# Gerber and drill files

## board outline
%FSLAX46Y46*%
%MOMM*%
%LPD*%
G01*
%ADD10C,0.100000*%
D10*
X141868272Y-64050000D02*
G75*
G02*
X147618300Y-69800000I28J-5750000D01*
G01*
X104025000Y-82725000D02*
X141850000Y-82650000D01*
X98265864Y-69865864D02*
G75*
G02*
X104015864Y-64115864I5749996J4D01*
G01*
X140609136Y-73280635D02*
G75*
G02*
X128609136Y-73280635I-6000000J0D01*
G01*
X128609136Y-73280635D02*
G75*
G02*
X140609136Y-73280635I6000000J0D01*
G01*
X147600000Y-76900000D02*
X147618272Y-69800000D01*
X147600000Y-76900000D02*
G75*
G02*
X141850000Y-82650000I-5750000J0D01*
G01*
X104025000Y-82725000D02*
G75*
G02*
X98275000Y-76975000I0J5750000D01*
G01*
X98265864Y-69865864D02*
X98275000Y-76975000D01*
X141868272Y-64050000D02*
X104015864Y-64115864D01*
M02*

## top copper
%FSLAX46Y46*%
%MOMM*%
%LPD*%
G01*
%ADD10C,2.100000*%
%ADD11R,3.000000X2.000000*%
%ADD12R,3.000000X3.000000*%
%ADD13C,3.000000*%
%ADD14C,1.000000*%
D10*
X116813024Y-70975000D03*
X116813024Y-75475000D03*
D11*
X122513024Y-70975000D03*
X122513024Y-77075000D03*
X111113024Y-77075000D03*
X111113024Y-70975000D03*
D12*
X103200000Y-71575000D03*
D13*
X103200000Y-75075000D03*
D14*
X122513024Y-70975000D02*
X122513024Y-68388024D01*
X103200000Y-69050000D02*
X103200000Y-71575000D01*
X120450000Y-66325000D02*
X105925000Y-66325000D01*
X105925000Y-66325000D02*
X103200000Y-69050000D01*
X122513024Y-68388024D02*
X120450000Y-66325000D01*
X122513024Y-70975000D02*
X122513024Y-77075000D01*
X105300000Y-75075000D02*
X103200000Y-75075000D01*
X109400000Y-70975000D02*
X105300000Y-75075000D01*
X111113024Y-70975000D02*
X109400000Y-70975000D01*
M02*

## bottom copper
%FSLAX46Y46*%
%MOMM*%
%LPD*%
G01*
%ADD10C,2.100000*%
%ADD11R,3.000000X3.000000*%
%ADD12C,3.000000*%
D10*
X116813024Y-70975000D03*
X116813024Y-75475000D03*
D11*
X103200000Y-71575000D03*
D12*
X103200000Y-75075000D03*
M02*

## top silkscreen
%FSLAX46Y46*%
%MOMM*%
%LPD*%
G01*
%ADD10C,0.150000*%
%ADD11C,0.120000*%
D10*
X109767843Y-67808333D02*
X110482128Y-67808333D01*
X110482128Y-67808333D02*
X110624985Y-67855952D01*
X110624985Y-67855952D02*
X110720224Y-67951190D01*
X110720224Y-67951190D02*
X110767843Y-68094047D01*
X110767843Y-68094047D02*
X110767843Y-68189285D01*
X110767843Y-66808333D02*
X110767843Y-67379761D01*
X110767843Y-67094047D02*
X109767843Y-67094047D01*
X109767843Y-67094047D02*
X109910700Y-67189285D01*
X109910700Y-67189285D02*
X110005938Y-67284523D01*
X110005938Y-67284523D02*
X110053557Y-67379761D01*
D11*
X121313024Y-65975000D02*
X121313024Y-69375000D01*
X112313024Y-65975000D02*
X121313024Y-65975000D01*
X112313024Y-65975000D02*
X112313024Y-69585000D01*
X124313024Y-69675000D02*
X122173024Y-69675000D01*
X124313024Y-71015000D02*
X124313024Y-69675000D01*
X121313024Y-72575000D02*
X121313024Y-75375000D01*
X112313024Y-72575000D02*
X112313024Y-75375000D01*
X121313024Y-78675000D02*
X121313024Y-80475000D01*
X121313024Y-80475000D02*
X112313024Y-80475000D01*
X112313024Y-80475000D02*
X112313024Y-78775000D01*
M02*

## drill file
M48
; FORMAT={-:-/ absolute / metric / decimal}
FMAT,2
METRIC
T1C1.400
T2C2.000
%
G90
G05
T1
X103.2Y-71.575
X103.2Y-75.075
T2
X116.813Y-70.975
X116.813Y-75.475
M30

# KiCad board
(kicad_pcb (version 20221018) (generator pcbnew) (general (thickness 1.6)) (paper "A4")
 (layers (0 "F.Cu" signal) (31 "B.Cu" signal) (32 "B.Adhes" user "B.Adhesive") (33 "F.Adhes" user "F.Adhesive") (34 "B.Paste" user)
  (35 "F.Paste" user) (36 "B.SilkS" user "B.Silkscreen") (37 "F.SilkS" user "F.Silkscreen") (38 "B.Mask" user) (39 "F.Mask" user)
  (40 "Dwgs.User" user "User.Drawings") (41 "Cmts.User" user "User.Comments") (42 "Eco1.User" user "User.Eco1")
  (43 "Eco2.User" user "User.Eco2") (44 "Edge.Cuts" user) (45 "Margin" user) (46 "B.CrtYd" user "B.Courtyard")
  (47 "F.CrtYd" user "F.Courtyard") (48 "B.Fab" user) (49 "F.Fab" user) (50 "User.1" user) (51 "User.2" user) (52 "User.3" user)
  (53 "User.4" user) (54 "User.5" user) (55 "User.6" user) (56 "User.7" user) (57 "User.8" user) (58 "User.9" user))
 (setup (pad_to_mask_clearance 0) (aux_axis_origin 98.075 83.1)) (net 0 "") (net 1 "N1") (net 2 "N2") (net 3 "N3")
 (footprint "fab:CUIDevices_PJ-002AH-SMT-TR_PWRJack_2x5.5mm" (layer "F.Cu") (at 116.813024 73.975 -90)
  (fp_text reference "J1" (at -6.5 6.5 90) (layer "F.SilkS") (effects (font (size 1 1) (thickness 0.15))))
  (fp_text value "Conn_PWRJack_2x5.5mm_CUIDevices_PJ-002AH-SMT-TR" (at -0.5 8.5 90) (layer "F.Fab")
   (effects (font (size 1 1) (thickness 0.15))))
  (fp_line (start -8 -4.5) (end -4.6 -4.5) (stroke (width 0.12) (type solid)) (layer "F.SilkS"))
  (fp_line (start -8 4.5) (end -8 -4.5) (stroke (width 0.12) (type solid)) (layer "F.SilkS"))
  (fp_line (start -8 4.5) (end -4.39 4.5) (stroke (width 0.12) (type solid)) (layer "F.SilkS"))
  (fp_line (start -4.3 -7.5) (end -4.3 -5.36) (stroke (width 0.12) (type solid)) (layer "F.SilkS"))
  (fp_line (start -2.96 -7.5) (end -4.3 -7.5) (stroke (width 0.12) (type solid)) (layer "F.SilkS"))
  (fp_line (start -1.4 -4.5) (end 1.4 -4.5) (stroke (width 0.12) (type solid)) (layer "F.SilkS"))
  (fp_line (start -1.4 4.5) (end 1.4 4.5) (stroke (width 0.12) (type solid)) (layer "F.SilkS"))
  (fp_line (start 4.7 -4.5) (end 6.5 -4.5) (stroke (width 0.12) (type solid)) (layer "F.SilkS"))
  (fp_line (start 6.5 -4.5) (end 6.5 4.5) (stroke (width 0.12) (type solid)) (layer "F.SilkS"))
  (fp_line (start 6.5 4.5) (end 4.8 4.5) (stroke (width 0.12) (type solid)) (layer "F.SilkS"))
  (pad "" thru_hole circle (at -3 0) (size 2.1 2.1) (drill 2) (layers "*.Cu" "*.Mask"))
  (pad "" thru_hole circle (at 1.5 0) (size 2.1 2.1) (drill 2) (layers "*.Cu" "*.Mask"))
  (pad "1" smd rect (at -3 -5.7) (size 3 2) (layers "F.Cu" "F.Paste" "F.Mask") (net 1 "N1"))
  (pad "1" smd rect (at 3.1 -5.7) (size 3 2) (layers "F.Cu" "F.Paste" "F.Mask") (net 1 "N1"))
  (pad "2" smd rect (at 3.1 5.7) (size 3 2) (layers "F.Cu" "F.Paste" "F.Mask") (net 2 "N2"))
  (pad "3" smd rect (at -3 5.7) (size 3 2) (layers "F.Cu" "F.Paste" "F.Mask") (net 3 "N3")))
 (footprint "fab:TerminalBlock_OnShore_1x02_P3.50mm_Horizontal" (layer "B.Cu") (at 103.2 71.575 -90)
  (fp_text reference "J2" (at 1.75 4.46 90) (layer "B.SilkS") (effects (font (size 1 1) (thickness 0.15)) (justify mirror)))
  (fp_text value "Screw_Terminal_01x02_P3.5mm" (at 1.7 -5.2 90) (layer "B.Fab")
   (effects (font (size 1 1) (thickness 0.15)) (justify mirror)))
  (pad "1" thru_hole rect (at 0 0 270) (size 3 3) (drill 1.4) (layers "*.Cu" "*.Mask") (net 1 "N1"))
  (pad "2" thru_hole circle (at 3.5 0 270) (size 3 3) (drill 1.4) (layers "*.Cu" "*.Mask") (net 3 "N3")))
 (gr_arc (start 141.868272 64.05) (mid 145.934136 65.734136) (end 147.618272 69.8) (stroke (width 0.1) (type default)) (layer "Edge.Cuts"))
 (gr_line (start 104.025 82.725) (end 141.85 82.65) (stroke (width 0.1) (type default)) (layer "Edge.Cuts"))
 (gr_arc (start 98.265864 69.865864) (mid 99.95 65.8) (end 104.015864 64.115864) (stroke (width 0.1) (type default)) (layer "Edge.Cuts"))
 (gr_circle (center 134.609136 73.280635) (end 140.609136 73.280635) (stroke (width 0.1) (type default)) (fill none) (layer "Edge.Cuts"))
 (gr_line (start 147.6 76.9) (end 147.618272 69.8) (stroke (width 0.1) (type default)) (layer "Edge.Cuts"))
 (gr_arc (start 147.6 76.9) (mid 145.915864 80.965864) (end 141.85 82.65) (stroke (width 0.1) (type default)) (layer "Edge.Cuts"))
 (gr_arc (start 104.025 82.725) (mid 99.959136 81.040864) (end 98.275 76.975) (stroke (width 0.1) (type default)) (layer "Edge.Cuts"))
 (gr_line (start 98.265864 69.865864) (end 98.275 76.975) (stroke (width 0.1) (type default)) (layer "Edge.Cuts"))
 (gr_line (start 141.868272 64.05) (end 104.015864 64.115864) (stroke (width 0.1) (type default)) (layer "Edge.Cuts"))
 (segment (start 122.513024 70.975) (end 122.513024 68.388024) (width 1) (layer "F.Cu") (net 1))
 (segment (start 103.2 69.05) (end 103.2 71.575) (width 1) (layer "F.Cu") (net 1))
 (segment (start 120.45 66.325) (end 105.925 66.325) (width 1) (layer "F.Cu") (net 1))
 (segment (start 105.925 66.325) (end 103.2 69.05) (width 1) (layer "F.Cu") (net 1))
 (segment (start 122.513024 68.388024) (end 120.45 66.325) (width 1) (layer "F.Cu") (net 1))
 (segment (start 122.513024 70.975) (end 122.513024 77.075) (width 1) (layer "F.Cu") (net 1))
 (segment (start 105.3 75.075) (end 103.2 75.075) (width 1) (layer "F.Cu") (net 3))
 (segment (start 109.4 70.975) (end 105.3 75.075) (width 1) (layer "F.Cu") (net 3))
 (segment (start 111.113024 70.975) (end 109.4 70.975) (width 1) (layer "F.Cu") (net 3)))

